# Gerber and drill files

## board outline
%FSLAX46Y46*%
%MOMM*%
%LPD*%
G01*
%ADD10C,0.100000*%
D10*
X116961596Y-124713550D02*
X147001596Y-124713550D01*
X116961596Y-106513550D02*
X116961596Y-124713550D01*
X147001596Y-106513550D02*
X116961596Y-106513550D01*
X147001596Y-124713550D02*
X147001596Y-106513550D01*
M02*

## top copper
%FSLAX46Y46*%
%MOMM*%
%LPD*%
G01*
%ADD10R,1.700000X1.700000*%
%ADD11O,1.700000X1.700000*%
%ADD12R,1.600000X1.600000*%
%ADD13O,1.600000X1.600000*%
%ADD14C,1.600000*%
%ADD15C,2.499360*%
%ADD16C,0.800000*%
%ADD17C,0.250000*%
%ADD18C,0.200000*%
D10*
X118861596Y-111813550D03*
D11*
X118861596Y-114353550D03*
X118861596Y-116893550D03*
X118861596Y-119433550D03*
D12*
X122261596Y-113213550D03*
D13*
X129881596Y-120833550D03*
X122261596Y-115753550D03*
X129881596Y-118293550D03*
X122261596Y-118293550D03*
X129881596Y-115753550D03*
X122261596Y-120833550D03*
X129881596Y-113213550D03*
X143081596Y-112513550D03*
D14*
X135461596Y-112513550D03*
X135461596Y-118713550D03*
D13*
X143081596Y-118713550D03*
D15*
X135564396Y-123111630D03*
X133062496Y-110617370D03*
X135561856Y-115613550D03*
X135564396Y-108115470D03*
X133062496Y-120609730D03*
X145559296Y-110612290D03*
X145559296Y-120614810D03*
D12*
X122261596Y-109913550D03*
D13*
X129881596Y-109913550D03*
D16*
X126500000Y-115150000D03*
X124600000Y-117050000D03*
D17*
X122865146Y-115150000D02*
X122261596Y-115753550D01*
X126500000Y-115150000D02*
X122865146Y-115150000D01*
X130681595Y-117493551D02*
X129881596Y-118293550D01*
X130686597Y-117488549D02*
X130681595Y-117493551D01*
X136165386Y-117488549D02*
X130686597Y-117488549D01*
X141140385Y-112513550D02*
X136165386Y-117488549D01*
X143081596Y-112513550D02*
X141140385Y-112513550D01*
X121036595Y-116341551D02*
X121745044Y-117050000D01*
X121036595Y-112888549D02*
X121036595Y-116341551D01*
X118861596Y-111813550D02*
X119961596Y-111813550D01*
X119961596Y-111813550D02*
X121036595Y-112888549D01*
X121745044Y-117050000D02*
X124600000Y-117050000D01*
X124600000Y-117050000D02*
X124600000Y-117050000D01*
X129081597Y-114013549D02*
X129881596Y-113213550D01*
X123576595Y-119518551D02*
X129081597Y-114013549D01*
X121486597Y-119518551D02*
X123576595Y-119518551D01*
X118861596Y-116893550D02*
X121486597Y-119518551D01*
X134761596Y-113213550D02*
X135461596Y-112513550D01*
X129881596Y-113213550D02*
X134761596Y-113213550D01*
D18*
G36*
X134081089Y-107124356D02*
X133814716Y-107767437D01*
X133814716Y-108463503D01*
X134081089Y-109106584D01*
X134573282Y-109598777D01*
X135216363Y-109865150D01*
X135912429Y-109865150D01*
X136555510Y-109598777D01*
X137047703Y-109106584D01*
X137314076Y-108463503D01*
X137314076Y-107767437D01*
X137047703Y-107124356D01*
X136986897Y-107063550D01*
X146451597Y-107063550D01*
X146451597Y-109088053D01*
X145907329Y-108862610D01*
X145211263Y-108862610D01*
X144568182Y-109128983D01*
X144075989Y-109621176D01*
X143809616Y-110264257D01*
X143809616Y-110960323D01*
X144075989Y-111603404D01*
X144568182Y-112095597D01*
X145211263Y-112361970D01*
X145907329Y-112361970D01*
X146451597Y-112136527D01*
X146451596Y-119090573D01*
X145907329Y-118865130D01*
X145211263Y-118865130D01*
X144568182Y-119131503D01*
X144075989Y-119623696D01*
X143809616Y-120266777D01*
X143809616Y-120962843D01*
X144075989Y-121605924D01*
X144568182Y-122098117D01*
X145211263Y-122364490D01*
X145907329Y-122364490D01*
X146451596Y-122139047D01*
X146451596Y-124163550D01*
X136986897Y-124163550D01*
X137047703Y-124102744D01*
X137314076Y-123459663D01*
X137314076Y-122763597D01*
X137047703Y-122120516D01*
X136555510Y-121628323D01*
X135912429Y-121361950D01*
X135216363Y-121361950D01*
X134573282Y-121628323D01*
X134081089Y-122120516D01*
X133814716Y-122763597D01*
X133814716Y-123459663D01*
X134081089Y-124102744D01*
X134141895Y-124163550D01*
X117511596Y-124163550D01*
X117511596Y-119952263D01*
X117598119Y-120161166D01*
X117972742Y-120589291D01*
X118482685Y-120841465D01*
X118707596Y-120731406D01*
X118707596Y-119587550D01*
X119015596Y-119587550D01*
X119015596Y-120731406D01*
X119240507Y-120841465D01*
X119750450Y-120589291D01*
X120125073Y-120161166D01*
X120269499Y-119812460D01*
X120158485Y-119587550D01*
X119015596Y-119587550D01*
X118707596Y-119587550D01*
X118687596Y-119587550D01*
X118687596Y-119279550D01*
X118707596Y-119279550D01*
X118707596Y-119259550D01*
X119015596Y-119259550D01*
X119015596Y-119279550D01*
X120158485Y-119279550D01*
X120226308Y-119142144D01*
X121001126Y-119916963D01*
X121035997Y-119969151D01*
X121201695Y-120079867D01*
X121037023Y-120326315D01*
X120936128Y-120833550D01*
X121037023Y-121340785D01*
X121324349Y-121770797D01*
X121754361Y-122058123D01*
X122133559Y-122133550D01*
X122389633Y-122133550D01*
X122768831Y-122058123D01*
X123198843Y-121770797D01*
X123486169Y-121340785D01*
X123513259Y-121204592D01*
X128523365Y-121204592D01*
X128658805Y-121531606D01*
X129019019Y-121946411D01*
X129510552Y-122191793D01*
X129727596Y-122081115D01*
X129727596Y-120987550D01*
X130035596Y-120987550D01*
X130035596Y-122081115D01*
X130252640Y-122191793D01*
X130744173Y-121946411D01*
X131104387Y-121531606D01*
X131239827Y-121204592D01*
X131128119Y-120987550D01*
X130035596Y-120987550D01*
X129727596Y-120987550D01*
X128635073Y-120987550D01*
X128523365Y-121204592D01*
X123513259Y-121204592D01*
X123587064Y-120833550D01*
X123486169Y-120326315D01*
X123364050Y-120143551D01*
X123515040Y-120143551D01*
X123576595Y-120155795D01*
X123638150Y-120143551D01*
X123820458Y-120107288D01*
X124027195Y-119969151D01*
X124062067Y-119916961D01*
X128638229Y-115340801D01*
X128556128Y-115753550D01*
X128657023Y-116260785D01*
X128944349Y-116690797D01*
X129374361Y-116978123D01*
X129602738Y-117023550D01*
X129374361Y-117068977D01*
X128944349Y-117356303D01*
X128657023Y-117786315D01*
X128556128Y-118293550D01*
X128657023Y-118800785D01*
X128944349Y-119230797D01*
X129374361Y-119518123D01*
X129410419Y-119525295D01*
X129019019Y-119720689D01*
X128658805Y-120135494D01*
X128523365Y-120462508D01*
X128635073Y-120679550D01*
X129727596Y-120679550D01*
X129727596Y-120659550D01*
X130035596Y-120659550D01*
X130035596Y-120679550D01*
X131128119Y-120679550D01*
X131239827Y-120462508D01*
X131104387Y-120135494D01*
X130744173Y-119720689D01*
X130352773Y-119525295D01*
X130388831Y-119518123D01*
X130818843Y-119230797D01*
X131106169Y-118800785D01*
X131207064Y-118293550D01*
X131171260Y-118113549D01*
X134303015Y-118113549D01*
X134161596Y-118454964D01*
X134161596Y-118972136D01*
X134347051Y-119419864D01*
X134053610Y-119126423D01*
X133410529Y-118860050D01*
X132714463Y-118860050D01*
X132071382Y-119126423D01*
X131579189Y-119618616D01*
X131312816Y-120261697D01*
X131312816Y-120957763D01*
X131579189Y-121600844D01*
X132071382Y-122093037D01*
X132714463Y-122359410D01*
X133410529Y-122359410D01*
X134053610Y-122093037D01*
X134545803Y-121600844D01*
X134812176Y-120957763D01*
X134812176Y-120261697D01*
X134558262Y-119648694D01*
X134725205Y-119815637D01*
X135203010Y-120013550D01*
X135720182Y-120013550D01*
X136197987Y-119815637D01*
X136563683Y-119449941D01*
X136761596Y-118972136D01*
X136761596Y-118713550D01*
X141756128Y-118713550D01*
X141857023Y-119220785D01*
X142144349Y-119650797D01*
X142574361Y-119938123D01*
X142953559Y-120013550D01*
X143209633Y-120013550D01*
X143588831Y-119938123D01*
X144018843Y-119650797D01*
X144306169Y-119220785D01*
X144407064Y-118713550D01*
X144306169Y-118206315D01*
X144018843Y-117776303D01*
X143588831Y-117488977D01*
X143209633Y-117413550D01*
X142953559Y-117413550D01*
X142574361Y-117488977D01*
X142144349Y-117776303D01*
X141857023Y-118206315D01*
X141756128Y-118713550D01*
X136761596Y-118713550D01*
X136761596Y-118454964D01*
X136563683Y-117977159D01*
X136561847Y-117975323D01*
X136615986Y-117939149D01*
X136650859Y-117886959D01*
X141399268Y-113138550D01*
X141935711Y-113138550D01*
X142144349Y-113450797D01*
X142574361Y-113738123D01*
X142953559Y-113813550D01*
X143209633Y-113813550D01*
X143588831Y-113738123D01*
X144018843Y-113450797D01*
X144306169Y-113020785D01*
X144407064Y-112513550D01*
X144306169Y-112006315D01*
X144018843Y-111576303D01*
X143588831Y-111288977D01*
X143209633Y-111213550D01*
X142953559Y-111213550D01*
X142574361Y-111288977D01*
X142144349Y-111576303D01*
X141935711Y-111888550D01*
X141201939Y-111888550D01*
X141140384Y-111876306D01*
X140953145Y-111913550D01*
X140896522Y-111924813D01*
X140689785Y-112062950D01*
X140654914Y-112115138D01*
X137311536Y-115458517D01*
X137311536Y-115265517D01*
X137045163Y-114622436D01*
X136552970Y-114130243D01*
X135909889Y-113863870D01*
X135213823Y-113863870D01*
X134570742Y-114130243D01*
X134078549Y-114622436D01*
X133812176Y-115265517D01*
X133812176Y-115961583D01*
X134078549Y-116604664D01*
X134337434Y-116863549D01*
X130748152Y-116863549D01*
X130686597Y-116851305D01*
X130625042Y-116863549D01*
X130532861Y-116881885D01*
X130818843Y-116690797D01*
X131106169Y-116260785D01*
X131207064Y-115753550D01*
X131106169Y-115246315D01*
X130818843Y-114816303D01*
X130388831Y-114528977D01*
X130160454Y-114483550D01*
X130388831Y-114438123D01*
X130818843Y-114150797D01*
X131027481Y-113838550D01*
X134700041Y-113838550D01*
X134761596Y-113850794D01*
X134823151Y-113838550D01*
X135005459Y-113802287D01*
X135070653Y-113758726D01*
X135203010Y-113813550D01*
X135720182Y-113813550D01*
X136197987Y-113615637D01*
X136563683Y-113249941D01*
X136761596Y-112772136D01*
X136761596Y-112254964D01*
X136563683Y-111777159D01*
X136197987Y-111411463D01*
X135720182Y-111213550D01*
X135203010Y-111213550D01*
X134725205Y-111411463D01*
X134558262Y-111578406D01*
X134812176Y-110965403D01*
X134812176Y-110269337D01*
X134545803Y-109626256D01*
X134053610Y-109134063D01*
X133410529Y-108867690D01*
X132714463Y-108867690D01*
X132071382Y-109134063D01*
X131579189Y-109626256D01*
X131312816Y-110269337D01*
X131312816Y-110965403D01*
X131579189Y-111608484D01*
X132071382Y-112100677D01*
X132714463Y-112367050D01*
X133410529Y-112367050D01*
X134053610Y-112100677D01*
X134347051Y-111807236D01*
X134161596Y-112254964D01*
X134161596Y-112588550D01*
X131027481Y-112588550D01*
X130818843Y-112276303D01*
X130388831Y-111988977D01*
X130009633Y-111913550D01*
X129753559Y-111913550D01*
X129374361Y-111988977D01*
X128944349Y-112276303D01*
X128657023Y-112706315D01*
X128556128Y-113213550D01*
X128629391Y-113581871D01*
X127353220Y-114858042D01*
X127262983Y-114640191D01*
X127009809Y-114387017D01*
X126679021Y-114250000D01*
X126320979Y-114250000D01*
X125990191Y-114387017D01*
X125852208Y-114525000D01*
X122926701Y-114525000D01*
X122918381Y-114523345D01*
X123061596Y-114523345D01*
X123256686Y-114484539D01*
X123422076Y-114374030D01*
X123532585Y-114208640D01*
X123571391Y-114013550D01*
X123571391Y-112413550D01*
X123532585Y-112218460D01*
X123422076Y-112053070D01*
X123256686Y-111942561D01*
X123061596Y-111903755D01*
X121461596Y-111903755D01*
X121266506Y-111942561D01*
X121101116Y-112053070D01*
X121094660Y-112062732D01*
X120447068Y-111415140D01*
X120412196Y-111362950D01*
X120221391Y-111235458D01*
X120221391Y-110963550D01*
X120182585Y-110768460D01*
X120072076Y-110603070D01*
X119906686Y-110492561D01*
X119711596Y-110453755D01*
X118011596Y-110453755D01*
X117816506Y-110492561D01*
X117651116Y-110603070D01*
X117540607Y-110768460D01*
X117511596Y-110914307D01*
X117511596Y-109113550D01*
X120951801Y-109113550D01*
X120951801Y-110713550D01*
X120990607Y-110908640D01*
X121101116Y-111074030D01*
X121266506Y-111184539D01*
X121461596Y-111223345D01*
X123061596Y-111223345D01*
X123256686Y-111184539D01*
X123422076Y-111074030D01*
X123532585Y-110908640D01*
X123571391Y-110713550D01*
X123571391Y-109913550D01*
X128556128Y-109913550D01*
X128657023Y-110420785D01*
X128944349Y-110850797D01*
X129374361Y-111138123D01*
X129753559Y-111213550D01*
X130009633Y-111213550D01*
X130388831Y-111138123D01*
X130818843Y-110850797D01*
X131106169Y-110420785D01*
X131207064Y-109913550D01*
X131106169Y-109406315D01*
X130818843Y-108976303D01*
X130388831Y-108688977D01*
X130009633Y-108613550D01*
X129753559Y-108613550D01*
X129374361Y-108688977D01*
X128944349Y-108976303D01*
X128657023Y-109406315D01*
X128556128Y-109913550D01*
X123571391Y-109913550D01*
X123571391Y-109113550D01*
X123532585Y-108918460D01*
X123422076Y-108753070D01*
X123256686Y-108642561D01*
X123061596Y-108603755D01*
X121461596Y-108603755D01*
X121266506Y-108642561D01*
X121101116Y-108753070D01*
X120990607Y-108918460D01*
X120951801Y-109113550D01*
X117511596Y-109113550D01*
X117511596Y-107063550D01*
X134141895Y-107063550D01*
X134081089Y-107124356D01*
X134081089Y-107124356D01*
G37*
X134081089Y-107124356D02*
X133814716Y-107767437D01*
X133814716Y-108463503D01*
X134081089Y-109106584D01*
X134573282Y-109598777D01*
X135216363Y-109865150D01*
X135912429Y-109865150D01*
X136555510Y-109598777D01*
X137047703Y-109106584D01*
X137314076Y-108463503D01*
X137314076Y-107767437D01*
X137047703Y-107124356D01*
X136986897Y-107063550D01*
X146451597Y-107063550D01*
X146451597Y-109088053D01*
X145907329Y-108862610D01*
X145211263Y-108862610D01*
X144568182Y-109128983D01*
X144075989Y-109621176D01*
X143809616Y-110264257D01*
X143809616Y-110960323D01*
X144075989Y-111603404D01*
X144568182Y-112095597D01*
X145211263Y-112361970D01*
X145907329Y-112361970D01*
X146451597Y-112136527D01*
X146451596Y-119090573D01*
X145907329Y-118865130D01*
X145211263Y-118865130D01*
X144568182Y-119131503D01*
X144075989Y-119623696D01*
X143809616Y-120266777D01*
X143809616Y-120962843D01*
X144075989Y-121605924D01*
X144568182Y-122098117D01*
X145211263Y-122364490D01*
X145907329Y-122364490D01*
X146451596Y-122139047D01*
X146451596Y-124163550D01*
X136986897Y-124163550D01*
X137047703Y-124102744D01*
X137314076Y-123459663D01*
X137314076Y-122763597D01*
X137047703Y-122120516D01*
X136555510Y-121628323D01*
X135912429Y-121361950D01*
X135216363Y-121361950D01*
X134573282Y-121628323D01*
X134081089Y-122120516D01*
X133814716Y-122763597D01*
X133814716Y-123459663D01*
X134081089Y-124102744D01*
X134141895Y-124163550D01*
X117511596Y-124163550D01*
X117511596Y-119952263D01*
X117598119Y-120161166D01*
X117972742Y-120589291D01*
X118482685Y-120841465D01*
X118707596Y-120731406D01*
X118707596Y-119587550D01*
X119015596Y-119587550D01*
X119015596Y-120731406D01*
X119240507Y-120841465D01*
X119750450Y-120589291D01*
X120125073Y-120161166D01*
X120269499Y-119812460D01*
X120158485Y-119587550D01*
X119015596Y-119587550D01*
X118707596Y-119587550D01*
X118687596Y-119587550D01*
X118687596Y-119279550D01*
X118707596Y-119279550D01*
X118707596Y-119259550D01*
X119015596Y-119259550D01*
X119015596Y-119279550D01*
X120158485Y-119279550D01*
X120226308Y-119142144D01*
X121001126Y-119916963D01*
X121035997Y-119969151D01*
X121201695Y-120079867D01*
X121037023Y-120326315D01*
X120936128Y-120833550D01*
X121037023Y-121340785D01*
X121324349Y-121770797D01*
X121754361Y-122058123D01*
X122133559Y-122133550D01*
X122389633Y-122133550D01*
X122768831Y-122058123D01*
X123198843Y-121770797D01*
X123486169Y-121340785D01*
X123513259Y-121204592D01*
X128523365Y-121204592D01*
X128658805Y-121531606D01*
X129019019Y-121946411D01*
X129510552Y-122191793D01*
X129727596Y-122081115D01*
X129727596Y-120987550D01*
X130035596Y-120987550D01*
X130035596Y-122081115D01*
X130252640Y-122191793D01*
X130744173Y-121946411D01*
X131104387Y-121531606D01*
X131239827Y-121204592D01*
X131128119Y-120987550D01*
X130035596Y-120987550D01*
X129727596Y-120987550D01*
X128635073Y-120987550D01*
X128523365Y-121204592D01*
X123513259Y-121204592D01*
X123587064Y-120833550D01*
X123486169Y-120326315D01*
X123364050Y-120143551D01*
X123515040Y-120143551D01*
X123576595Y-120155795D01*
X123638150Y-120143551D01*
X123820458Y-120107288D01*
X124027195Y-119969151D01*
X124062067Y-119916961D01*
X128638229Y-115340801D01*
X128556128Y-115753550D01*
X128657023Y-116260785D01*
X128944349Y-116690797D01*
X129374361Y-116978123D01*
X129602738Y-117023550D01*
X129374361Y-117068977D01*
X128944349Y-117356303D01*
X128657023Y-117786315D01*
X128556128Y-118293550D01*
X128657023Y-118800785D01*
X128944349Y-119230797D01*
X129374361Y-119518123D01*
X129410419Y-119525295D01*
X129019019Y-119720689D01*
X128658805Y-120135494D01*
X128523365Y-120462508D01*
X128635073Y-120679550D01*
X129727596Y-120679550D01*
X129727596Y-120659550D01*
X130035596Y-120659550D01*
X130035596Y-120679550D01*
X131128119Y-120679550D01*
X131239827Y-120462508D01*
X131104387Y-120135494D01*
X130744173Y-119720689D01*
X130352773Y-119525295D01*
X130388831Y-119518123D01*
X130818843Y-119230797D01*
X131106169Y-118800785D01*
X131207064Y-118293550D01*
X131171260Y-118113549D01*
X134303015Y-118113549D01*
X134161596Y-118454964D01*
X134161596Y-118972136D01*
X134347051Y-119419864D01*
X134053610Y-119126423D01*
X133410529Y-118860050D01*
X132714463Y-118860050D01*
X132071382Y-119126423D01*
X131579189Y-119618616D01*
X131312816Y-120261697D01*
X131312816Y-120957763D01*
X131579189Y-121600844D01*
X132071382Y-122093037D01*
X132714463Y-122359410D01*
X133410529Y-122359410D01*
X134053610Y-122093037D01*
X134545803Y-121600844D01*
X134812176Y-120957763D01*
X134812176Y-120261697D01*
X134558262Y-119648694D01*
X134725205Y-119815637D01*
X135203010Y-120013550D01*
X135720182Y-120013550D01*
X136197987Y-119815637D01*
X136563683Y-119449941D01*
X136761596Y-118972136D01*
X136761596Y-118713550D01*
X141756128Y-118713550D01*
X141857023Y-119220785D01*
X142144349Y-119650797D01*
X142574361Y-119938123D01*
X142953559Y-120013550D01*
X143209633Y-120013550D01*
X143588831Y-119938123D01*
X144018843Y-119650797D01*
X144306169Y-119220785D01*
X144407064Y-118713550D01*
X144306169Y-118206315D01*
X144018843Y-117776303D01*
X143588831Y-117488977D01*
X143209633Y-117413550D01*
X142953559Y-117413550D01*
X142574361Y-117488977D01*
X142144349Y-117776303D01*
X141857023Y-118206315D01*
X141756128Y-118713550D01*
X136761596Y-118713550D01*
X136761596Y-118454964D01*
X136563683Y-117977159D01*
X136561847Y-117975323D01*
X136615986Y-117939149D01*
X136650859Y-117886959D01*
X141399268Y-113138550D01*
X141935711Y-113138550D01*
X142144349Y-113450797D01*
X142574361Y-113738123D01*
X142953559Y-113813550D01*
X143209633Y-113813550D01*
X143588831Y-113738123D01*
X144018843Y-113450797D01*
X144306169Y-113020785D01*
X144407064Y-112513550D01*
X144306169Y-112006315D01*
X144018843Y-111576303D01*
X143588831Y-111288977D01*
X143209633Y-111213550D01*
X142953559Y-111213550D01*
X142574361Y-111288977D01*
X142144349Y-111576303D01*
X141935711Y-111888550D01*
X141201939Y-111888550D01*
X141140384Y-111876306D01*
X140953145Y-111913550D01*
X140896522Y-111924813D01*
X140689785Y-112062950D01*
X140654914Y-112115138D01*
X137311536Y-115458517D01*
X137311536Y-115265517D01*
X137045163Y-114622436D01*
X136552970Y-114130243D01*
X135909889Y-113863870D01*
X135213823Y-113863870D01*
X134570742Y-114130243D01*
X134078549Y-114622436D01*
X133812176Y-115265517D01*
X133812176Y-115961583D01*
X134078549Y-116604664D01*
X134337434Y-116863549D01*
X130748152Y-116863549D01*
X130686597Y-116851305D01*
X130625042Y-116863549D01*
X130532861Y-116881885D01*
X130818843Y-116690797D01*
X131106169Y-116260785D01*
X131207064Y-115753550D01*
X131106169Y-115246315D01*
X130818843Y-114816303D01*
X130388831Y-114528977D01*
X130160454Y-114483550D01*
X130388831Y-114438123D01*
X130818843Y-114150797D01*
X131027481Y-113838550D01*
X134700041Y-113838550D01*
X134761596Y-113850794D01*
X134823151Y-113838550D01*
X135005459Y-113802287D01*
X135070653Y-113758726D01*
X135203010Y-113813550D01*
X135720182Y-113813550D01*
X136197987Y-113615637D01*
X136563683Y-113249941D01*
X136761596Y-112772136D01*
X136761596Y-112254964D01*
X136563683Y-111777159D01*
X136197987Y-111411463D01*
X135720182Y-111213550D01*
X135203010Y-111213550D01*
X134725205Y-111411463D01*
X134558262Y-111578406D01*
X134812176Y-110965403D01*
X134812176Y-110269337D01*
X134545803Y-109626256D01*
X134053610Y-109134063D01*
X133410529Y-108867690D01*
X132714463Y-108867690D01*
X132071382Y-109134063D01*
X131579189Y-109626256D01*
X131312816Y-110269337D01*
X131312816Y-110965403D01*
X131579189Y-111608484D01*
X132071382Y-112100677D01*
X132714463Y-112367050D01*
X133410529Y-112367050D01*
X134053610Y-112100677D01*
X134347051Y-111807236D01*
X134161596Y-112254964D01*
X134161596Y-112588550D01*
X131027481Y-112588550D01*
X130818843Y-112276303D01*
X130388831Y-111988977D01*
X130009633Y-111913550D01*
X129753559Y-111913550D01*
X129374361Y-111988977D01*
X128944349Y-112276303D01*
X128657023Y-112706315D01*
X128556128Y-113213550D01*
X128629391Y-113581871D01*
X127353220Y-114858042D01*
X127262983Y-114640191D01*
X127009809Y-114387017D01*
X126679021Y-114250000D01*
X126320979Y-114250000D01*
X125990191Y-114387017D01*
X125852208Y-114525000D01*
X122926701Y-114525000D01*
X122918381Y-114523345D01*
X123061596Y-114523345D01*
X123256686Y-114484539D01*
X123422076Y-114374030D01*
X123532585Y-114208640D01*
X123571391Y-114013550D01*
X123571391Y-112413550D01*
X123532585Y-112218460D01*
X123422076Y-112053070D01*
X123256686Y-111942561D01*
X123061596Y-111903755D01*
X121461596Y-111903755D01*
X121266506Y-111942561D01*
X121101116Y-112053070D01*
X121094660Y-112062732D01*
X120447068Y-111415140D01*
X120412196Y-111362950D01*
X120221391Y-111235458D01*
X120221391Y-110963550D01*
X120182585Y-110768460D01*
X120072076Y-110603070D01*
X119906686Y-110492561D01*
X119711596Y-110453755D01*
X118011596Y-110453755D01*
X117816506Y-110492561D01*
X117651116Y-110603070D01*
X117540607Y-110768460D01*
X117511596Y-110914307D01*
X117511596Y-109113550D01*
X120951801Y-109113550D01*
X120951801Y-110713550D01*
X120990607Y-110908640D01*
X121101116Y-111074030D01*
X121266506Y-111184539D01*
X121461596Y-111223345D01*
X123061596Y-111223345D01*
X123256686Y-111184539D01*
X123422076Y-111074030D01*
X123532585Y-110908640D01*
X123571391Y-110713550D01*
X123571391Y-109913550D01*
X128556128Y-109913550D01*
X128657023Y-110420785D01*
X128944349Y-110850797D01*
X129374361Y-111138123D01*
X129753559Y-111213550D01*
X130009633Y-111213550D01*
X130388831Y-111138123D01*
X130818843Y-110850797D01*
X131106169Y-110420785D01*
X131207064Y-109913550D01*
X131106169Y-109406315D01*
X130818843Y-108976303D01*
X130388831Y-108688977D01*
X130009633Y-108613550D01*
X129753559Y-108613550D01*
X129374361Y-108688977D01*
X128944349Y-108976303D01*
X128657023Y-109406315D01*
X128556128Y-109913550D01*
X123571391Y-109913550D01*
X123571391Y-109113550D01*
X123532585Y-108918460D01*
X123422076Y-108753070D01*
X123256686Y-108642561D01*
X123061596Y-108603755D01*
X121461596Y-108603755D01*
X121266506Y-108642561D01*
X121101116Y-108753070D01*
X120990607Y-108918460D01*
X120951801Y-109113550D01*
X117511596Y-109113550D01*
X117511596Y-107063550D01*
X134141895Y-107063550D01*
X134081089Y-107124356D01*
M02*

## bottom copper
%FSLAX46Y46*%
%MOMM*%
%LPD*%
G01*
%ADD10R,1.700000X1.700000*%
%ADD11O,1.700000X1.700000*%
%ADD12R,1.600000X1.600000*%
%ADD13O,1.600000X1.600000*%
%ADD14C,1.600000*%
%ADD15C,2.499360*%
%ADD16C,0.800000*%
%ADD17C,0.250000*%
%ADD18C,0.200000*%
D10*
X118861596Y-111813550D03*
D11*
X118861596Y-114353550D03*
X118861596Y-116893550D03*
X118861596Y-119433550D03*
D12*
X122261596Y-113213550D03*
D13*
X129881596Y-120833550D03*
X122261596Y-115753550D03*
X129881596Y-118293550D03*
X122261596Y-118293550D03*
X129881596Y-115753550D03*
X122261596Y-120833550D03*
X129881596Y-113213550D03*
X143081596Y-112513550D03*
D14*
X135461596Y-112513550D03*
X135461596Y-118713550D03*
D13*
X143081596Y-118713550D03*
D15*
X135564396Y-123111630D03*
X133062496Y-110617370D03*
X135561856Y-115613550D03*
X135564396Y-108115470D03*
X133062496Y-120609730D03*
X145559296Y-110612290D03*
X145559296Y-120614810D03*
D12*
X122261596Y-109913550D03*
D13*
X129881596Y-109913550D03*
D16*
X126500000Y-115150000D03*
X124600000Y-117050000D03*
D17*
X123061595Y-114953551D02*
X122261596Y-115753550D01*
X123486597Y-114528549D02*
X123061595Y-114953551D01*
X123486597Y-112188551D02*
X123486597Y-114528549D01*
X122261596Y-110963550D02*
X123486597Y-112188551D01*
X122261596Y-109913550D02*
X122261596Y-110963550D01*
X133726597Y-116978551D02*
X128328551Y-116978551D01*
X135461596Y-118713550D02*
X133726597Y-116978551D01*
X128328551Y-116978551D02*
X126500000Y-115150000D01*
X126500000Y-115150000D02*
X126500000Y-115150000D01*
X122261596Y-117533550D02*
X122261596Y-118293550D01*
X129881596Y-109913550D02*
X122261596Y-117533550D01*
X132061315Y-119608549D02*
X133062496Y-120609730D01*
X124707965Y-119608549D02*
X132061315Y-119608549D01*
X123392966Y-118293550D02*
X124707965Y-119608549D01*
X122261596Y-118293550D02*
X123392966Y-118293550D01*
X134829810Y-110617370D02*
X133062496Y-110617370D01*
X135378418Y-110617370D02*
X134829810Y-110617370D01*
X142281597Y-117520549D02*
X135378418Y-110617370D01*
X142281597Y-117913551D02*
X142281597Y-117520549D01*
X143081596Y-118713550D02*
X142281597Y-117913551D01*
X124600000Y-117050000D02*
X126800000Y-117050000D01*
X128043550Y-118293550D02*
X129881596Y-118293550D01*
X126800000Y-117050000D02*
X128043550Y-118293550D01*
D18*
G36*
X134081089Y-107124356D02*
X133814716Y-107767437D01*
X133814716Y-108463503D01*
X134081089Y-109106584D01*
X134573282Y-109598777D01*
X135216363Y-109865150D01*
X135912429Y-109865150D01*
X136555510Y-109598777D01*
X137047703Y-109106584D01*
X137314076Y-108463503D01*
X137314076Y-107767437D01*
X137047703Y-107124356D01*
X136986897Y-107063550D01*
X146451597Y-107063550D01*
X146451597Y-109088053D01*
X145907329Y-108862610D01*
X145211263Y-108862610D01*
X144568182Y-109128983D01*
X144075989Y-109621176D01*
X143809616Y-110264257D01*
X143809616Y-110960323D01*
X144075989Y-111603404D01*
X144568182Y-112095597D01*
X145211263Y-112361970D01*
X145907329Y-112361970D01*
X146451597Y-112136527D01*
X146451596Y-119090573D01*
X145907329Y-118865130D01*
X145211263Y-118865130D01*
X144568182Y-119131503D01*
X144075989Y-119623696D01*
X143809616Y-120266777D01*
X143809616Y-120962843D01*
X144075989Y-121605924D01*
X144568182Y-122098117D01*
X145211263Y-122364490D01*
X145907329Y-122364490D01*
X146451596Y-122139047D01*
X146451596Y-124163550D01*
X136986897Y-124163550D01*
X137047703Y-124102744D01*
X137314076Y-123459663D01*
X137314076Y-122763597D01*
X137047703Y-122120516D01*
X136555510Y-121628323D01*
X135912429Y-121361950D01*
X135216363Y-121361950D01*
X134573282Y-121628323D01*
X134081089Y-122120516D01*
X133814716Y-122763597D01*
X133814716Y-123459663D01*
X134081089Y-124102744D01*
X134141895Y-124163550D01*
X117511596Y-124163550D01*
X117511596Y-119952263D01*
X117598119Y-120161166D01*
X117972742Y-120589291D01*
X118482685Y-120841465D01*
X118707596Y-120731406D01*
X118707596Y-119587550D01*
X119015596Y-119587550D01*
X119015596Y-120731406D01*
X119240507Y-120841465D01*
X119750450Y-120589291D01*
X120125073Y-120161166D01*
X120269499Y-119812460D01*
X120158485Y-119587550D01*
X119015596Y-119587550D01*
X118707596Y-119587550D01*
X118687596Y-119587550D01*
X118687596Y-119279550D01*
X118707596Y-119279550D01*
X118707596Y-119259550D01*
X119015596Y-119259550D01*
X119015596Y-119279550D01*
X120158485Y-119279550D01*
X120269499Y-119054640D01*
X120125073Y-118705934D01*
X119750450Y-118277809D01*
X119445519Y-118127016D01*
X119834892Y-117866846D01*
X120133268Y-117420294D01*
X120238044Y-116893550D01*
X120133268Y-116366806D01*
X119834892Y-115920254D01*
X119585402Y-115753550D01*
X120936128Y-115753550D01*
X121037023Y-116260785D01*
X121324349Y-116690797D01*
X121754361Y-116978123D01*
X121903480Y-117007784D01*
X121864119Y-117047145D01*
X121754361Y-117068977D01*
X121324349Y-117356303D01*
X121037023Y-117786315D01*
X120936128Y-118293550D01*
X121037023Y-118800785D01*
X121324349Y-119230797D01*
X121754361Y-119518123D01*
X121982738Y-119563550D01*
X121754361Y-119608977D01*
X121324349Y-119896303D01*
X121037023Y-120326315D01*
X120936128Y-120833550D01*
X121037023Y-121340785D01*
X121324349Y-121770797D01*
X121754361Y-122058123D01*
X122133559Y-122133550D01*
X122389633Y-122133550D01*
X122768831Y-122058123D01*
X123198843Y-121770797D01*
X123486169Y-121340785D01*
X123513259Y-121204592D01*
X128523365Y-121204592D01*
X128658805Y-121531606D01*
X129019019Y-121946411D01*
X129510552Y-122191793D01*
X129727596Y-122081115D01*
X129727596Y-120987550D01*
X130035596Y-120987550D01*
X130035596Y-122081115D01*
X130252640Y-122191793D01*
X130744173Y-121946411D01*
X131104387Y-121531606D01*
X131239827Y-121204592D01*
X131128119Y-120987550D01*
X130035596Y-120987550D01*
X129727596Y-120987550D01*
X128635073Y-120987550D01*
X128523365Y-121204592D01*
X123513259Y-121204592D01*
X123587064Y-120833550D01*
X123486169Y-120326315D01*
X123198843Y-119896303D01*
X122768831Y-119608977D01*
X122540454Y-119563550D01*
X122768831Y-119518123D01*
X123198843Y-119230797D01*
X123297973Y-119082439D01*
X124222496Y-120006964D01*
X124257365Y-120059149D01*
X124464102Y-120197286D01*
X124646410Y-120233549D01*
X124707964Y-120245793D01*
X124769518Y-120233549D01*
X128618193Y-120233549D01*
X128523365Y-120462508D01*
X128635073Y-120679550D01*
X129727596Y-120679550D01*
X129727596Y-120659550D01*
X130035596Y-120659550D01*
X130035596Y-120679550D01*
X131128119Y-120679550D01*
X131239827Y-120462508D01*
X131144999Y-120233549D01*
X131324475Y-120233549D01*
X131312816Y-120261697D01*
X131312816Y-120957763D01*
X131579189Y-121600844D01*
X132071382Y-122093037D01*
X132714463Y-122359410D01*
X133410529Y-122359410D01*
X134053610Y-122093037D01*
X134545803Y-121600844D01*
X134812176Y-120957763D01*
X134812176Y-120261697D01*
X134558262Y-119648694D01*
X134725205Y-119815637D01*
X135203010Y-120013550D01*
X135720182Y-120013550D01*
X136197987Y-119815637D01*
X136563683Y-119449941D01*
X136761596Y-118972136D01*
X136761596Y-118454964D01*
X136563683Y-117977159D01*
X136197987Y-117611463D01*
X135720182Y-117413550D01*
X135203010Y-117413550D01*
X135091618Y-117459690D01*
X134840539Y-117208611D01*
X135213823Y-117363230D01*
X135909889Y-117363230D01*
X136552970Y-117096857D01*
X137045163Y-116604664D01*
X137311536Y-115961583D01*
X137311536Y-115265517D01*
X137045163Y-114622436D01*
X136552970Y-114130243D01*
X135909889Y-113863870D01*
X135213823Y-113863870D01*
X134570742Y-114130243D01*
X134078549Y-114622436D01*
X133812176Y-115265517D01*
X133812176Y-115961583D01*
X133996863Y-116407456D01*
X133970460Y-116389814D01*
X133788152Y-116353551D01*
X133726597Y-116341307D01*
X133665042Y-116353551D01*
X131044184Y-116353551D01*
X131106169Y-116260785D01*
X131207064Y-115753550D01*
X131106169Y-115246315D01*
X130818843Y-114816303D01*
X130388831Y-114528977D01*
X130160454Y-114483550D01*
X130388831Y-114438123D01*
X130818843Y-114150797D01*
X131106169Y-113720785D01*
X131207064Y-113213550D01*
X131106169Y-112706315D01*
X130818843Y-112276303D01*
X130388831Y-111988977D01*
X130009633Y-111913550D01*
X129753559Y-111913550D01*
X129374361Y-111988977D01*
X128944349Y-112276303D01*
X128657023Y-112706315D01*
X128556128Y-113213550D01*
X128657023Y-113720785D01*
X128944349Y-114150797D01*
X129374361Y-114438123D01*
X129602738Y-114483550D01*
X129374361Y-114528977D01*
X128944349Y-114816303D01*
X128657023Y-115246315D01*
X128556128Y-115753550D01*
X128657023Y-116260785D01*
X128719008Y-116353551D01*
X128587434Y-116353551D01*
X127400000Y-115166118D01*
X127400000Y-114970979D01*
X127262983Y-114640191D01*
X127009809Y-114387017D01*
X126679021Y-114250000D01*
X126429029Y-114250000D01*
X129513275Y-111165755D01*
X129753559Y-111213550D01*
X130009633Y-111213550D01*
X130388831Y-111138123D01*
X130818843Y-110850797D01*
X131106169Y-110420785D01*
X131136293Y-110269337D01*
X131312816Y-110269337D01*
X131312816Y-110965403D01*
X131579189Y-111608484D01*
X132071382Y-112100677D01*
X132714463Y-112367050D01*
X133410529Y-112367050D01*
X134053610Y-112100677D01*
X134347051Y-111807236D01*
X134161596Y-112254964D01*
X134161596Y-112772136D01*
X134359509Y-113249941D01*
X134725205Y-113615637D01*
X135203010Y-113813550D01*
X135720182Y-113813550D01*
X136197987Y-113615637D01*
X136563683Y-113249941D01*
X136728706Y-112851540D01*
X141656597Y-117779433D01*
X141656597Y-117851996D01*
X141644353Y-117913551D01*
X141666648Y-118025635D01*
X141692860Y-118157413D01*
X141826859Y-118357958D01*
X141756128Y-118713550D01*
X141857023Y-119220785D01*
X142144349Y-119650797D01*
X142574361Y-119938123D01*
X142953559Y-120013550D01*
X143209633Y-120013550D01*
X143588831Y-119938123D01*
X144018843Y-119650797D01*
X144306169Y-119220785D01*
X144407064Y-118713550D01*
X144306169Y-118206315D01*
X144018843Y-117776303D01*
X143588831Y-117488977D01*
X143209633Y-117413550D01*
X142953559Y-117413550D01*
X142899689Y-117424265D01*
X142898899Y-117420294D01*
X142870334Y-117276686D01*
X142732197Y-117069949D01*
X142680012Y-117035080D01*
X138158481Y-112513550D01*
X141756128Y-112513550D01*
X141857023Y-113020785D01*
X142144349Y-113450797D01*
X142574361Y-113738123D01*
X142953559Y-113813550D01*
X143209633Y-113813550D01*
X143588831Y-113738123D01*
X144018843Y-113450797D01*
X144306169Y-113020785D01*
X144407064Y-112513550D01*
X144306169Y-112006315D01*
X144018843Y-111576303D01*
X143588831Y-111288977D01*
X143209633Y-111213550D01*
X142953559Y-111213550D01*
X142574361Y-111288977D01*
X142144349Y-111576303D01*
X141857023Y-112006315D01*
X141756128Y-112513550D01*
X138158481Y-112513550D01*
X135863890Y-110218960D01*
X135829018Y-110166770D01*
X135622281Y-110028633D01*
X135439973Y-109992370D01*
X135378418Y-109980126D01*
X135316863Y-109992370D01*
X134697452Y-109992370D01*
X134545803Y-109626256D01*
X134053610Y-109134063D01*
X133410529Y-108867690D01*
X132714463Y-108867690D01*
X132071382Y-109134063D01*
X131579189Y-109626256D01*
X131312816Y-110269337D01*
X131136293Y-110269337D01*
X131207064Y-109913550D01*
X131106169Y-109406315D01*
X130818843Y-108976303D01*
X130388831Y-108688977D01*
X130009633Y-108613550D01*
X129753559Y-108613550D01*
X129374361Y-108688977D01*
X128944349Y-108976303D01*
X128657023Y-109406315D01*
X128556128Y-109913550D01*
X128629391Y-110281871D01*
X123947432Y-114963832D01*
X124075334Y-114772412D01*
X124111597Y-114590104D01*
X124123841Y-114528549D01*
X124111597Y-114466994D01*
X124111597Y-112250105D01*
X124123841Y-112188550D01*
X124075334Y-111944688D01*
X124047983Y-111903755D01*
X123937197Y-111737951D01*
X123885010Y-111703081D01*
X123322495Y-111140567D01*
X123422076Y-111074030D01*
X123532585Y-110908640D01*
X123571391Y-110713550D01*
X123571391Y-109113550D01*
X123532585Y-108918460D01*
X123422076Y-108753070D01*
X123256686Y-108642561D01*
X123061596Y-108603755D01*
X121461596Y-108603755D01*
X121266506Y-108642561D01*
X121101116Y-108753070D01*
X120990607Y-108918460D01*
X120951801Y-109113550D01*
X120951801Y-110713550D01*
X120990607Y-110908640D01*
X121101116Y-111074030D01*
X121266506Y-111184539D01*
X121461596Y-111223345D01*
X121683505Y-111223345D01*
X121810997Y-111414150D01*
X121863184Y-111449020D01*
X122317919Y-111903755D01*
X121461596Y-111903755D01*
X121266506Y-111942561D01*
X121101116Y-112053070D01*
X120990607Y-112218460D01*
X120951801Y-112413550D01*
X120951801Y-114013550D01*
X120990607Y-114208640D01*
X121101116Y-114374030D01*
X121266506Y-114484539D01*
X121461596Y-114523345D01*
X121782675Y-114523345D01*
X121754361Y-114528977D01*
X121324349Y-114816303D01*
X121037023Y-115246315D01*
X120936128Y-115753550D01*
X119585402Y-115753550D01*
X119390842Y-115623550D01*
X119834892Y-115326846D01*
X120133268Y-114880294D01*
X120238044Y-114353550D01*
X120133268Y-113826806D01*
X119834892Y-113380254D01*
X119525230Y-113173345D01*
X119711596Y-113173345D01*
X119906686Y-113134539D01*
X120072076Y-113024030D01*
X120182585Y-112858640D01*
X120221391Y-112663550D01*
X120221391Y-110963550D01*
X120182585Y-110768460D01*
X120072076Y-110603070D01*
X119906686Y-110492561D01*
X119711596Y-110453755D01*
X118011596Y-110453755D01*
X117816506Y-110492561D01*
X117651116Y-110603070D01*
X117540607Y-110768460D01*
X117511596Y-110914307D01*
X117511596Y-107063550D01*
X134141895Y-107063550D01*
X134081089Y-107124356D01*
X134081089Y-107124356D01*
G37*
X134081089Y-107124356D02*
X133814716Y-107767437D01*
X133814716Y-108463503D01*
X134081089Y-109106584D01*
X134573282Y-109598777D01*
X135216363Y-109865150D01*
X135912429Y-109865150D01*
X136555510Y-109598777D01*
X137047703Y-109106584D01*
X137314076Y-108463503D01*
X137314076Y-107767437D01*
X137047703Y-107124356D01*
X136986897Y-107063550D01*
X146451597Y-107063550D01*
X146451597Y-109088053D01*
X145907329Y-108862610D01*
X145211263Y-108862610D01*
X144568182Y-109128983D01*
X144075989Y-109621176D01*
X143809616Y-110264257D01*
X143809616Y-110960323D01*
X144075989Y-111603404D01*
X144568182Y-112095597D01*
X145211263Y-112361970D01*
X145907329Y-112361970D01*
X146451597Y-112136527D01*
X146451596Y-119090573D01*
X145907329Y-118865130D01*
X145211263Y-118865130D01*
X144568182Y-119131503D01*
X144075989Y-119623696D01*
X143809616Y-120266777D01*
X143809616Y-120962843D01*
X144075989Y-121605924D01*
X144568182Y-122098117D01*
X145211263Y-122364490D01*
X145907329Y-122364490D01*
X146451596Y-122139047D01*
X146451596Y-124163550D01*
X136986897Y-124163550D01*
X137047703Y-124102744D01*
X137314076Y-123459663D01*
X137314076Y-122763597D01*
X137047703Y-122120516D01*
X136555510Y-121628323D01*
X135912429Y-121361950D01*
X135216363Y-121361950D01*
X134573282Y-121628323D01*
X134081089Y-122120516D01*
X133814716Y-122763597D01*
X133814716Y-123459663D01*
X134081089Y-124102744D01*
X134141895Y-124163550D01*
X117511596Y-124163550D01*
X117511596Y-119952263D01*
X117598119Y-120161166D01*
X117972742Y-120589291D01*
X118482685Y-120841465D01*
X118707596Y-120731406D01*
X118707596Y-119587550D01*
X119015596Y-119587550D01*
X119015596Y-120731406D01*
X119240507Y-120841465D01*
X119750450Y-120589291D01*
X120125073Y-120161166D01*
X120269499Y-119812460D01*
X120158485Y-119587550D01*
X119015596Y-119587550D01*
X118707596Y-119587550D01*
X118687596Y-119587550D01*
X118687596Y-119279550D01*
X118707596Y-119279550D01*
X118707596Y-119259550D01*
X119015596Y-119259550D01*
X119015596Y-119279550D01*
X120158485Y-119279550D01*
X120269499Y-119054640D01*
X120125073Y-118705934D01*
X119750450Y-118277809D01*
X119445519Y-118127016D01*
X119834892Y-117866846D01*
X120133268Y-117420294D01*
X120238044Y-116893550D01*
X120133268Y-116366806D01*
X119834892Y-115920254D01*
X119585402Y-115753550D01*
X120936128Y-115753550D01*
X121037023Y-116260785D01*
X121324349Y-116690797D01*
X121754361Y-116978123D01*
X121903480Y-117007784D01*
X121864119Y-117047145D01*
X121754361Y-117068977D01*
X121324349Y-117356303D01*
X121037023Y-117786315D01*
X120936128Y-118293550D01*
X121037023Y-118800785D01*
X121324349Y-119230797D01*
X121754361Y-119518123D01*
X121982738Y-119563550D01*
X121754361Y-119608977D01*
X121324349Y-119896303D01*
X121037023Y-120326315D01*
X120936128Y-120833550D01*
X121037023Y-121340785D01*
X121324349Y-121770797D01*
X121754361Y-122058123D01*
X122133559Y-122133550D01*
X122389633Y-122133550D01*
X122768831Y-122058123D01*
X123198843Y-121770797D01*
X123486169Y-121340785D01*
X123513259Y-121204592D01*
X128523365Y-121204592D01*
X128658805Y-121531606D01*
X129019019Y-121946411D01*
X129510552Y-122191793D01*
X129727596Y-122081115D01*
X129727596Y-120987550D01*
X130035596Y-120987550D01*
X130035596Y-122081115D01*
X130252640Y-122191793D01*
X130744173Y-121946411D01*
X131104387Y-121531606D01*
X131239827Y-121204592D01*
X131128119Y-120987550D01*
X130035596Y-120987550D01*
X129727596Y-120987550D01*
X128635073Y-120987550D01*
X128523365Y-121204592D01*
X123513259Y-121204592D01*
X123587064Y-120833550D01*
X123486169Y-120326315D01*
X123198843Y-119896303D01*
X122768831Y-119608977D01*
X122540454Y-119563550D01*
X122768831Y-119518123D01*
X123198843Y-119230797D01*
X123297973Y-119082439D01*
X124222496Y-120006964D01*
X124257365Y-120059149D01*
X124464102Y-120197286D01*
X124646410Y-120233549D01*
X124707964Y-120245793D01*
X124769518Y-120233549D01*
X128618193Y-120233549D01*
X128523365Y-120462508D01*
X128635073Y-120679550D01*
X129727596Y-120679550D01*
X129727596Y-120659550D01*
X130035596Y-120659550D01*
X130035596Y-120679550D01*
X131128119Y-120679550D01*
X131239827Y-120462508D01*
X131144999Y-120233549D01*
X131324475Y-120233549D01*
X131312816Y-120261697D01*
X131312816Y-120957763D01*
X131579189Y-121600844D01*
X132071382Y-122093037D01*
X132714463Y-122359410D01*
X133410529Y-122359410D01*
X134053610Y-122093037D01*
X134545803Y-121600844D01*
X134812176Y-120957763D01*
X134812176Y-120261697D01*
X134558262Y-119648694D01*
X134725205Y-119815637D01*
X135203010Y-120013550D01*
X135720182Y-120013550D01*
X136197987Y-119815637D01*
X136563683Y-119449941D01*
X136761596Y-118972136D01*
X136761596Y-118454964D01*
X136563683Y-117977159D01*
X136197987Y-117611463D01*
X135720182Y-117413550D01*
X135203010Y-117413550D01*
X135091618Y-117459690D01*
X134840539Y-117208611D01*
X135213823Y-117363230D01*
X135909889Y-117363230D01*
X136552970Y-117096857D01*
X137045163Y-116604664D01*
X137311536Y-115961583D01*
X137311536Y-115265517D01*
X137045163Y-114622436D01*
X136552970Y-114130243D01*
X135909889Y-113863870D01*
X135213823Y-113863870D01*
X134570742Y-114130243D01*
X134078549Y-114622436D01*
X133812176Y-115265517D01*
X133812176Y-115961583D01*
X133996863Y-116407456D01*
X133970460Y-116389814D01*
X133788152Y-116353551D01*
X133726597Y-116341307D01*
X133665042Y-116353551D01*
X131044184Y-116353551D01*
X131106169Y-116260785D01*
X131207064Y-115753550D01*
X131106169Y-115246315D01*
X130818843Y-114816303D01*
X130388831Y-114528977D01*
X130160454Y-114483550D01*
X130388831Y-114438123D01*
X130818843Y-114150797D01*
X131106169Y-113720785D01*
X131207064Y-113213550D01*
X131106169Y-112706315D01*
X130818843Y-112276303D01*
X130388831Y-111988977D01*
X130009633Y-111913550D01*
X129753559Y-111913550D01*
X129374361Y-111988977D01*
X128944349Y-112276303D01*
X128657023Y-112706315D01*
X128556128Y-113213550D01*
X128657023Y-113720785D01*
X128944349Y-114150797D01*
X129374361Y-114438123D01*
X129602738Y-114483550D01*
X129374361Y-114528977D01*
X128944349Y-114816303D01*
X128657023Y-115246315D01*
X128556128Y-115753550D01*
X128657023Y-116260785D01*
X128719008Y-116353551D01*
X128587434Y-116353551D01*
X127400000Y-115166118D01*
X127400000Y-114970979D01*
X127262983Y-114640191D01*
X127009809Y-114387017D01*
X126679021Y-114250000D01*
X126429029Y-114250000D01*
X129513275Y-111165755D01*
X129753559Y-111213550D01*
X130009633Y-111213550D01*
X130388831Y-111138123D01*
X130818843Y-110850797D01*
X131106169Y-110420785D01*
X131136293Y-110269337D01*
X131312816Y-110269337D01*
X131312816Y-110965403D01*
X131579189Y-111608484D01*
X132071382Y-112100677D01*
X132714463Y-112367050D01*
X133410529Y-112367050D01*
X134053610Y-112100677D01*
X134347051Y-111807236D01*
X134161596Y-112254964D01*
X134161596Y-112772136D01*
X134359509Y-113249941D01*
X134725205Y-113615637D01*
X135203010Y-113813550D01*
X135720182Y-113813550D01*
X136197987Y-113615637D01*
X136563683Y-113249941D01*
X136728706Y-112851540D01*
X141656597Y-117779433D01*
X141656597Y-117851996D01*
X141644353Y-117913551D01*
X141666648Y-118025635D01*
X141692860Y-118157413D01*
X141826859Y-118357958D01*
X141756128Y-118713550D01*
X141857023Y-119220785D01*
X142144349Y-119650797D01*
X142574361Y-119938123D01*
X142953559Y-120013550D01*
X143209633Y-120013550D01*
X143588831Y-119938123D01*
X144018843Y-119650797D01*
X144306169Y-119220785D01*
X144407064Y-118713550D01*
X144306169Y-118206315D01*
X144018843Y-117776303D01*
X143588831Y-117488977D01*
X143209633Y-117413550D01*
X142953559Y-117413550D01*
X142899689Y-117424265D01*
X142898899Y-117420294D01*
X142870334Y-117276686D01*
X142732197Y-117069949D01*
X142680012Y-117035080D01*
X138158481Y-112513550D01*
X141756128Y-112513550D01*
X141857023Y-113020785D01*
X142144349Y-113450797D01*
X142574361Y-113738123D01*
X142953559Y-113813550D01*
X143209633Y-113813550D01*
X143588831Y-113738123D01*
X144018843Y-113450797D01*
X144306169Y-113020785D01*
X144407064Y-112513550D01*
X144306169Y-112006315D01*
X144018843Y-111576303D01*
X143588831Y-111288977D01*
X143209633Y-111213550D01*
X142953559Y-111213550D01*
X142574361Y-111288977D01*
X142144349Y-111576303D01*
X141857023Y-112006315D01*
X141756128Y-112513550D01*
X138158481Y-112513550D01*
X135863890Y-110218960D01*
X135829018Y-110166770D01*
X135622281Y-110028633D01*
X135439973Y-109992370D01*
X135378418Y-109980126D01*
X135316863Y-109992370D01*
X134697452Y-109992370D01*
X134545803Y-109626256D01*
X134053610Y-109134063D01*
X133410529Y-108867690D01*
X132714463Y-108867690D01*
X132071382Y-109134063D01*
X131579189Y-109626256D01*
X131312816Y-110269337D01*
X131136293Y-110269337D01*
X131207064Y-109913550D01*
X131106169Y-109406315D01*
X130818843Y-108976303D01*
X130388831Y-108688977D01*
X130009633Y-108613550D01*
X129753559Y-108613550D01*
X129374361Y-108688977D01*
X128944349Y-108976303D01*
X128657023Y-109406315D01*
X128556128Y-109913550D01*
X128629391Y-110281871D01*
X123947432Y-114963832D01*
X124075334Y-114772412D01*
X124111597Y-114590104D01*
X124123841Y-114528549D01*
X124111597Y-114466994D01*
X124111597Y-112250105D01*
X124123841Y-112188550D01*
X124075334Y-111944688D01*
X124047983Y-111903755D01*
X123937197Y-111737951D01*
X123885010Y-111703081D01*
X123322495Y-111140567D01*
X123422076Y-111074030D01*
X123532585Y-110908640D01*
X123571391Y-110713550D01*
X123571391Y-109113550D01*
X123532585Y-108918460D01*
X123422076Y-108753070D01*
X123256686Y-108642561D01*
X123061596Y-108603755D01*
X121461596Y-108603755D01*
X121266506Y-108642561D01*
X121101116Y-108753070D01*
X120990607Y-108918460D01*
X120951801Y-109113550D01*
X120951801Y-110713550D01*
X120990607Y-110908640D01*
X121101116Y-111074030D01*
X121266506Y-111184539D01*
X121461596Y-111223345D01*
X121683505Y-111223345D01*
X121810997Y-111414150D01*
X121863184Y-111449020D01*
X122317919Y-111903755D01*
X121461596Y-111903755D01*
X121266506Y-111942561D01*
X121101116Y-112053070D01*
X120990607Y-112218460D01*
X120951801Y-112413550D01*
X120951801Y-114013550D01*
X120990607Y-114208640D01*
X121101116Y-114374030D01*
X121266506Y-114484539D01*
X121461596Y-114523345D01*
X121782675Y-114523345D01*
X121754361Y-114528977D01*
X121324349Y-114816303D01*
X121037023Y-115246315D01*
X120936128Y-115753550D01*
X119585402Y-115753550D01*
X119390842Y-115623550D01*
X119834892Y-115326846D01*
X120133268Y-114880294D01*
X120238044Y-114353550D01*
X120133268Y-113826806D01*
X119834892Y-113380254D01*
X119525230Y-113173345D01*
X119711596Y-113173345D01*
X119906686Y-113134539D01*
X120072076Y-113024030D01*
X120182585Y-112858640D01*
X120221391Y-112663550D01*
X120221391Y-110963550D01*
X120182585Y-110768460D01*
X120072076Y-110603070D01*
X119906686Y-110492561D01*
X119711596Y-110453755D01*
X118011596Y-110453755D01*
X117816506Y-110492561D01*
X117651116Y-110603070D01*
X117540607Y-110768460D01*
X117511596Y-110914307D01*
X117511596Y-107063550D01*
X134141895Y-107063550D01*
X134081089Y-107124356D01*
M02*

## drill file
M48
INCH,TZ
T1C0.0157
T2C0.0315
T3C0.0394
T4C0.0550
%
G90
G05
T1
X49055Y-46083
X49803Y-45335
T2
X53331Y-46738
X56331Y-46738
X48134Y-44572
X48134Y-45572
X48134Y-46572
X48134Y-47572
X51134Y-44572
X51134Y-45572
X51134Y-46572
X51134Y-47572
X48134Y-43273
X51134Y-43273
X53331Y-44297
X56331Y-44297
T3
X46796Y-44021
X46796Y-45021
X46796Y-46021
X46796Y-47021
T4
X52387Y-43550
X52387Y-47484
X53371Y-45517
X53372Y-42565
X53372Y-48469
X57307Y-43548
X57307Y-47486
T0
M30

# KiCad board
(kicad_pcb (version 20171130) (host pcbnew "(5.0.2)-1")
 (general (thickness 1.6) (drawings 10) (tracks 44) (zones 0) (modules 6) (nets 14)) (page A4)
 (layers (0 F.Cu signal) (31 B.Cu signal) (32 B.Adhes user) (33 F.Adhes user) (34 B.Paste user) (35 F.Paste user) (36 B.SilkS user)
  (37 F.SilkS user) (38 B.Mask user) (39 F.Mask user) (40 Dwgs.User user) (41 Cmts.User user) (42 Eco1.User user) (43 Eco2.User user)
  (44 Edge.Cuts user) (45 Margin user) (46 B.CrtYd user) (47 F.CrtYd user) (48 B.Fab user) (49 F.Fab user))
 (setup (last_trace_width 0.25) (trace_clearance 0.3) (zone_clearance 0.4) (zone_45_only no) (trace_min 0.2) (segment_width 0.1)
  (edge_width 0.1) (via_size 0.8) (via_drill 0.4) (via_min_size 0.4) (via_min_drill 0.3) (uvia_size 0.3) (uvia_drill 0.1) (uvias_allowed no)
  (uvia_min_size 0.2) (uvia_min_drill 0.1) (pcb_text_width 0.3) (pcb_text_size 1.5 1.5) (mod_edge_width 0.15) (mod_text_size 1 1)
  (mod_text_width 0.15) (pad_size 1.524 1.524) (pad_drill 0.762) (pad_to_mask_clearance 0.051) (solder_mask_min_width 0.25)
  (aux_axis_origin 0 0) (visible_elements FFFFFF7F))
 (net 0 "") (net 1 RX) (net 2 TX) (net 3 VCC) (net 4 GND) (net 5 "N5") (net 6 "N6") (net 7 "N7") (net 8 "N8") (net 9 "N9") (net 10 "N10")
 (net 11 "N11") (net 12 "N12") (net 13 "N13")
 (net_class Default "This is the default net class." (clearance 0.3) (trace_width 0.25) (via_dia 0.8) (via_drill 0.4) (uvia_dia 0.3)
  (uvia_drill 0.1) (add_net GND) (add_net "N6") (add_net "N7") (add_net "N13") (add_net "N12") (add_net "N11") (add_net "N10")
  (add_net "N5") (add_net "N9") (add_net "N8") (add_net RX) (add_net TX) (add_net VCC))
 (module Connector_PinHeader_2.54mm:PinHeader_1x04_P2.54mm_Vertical (layer F.Cu) (at 118.861596 111.81355)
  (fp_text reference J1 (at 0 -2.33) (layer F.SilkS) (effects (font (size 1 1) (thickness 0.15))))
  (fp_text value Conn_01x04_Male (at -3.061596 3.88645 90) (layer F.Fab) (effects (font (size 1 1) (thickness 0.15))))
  (pad 1 thru_hole rect (at 0 0) (size 1.7 1.7) (drill 1) (layers *.Cu *.Mask) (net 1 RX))
  (pad 2 thru_hole oval (at 0 2.54) (size 1.7 1.7) (drill 1) (layers *.Cu *.Mask) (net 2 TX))
  (pad 3 thru_hole oval (at 0 5.08) (size 1.7 1.7) (drill 1) (layers *.Cu *.Mask) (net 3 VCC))
  (pad 4 thru_hole oval (at 0 7.62) (size 1.7 1.7) (drill 1) (layers *.Cu *.Mask) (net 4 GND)))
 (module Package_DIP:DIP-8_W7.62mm (layer F.Cu) (at 122.261596 113.21355)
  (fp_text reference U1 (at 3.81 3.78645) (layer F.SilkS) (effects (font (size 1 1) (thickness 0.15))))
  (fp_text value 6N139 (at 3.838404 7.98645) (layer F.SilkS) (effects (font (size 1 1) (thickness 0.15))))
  (pad 1 thru_hole rect (at 0 0) (size 1.6 1.6) (drill 0.8) (layers *.Cu *.Mask) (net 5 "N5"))
  (pad 5 thru_hole oval (at 7.62 7.62) (size 1.6 1.6) (drill 0.8) (layers *.Cu *.Mask) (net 4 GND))
  (pad 2 thru_hole oval (at 0 2.54) (size 1.6 1.6) (drill 0.8) (layers *.Cu *.Mask) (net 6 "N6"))
  (pad 6 thru_hole oval (at 7.62 5.08) (size 1.6 1.6) (drill 0.8) (layers *.Cu *.Mask) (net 1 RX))
  (pad 3 thru_hole oval (at 0 5.08) (size 1.6 1.6) (drill 0.8) (layers *.Cu *.Mask) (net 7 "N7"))
  (pad 7 thru_hole oval (at 7.62 2.54) (size 1.6 1.6) (drill 0.8) (layers *.Cu *.Mask) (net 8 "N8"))
  (pad 4 thru_hole oval (at 0 7.62) (size 1.6 1.6) (drill 0.8) (layers *.Cu *.Mask) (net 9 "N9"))
  (pad 8 thru_hole oval (at 7.62 0) (size 1.6 1.6) (drill 0.8) (layers *.Cu *.Mask) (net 3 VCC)))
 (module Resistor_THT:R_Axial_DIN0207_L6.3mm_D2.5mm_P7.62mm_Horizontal (layer B.Cu) (at 135.461596 112.51355)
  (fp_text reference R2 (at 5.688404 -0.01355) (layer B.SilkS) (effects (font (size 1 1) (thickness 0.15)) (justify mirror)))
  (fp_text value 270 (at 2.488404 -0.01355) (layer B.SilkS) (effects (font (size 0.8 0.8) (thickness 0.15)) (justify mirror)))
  (pad 2 thru_hole oval (at 7.62 0) (size 1.6 1.6) (drill 0.8) (layers *.Cu *.Mask) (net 1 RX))
  (pad 1 thru_hole circle (at 0 0) (size 1.6 1.6) (drill 0.8) (layers *.Cu *.Mask) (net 3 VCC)))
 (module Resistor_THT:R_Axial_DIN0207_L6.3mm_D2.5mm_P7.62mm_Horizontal (layer B.Cu) (at 135.461596 118.71355)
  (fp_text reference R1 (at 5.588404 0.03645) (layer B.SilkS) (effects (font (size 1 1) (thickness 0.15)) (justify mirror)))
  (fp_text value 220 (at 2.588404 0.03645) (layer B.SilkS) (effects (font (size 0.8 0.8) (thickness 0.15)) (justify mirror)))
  (pad 1 thru_hole circle (at 0 0) (size 1.6 1.6) (drill 0.8) (layers *.Cu *.Mask) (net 6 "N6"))
  (pad 2 thru_hole oval (at 7.62 0) (size 1.6 1.6) (drill 0.8) (layers *.Cu *.Mask) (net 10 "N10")))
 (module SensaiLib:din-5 (layer F.Cu) (at 138.561596 115.61355 90)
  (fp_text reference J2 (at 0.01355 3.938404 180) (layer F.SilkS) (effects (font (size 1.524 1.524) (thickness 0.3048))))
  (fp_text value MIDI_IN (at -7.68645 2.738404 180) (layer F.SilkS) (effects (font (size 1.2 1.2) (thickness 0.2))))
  (pad 3 thru_hole circle (at -7.49808 -2.9972 90) (size 2.49936 2.49936) (drill 1.397) (layers *.Cu *.SilkS *.Mask) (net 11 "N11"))
  (pad 4 thru_hole circle (at 4.99618 -5.4991 90) (size 2.49936 2.49936) (drill 1.397) (layers *.Cu *.SilkS *.Mask) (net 10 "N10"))
  (pad 2 thru_hole circle (at 0 -2.99974 90) (size 2.49936 2.49936) (drill 1.397) (layers *.Cu *.SilkS *.Mask) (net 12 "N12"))
  (pad 1 thru_hole circle (at 7.49808 -2.9972 90) (size 2.49936 2.49936) (drill 1.397) (layers *.Cu *.SilkS *.Mask) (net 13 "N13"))
  (pad 5 thru_hole circle (at -4.99618 -5.4991 90) (size 2.49936 2.49936) (drill 1.397) (layers *.Cu *.SilkS *.Mask) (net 7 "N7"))
  (pad "" thru_hole circle (at 5.00126 6.9977 90) (size 2.49936 2.49936) (drill 1.397) (layers *.Cu *.Mask))
  (pad "" thru_hole circle (at -5.00126 6.9977 90) (size 2.49936 2.49936) (drill 1.397) (layers *.Cu *.Mask)))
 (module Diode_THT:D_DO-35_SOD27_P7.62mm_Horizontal (layer F.Cu) (at 122.261596 109.91355)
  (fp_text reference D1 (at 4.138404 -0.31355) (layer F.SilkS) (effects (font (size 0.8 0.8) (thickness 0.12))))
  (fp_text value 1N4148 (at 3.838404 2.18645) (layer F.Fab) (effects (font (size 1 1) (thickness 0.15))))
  (pad 1 thru_hole rect (at 0 0) (size 1.6 1.6) (drill 0.8) (layers *.Cu *.Mask) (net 6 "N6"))
  (pad 2 thru_hole oval (at 7.62 0) (size 1.6 1.6) (drill 0.8) (layers *.Cu *.Mask) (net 7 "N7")))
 (gr_line (start 116.961596 124.71355) (end 147.001596 124.71355) (layer Edge.Cuts) (width 0.1))
 (gr_line (start 116.961596 106.51355) (end 116.961596 124.71355) (layer Edge.Cuts) (width 0.1))
 (gr_line (start 147.001596 106.51355) (end 116.961596 106.51355) (layer Edge.Cuts) (width 0.1))
 (gr_line (start 147.001596 124.71355) (end 147.001596 106.51355) (layer Edge.Cuts) (width 0.1))
 (segment (start 123.061595 114.953551) (end 122.261596 115.75355) (width 0.25) (layer B.Cu) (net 6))
 (segment (start 123.486597 114.528549) (end 123.061595 114.953551) (width 0.25) (layer B.Cu) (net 6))
 (segment (start 123.486597 112.188551) (end 123.486597 114.528549) (width 0.25) (layer B.Cu) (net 6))
 (segment (start 122.261596 110.96355) (end 123.486597 112.188551) (width 0.25) (layer B.Cu) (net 6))
 (segment (start 122.261596 109.91355) (end 122.261596 110.96355) (width 0.25) (layer B.Cu) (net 6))
 (segment (start 133.726597 116.978551) (end 128.328551 116.978551) (width 0.25) (layer B.Cu) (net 6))
 (segment (start 135.461596 118.71355) (end 133.726597 116.978551) (width 0.25) (layer B.Cu) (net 6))
 (segment (start 128.328551 116.978551) (end 126.5 115.15) (width 0.25) (layer B.Cu) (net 6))
 (segment (start 126.5 115.15) (end 126.5 115.15) (width 0.25) (layer B.Cu) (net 6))
 (via (at 126.5 115.15) (size 0.8) (drill 0.4) (layers F.Cu B.Cu) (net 6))
 (segment (start 122.865146 115.15) (end 122.261596 115.75355) (width 0.25) (layer F.Cu) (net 6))
 (segment (start 126.5 115.15) (end 122.865146 115.15) (width 0.25) (layer F.Cu) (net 6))
 (segment (start 122.261596 117.53355) (end 122.261596 118.29355) (width 0.25) (layer B.Cu) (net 7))
 (segment (start 129.881596 109.91355) (end 122.261596 117.53355) (width 0.25) (layer B.Cu) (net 7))
 (segment (start 132.061315 119.608549) (end 133.062496 120.60973) (width 0.25) (layer B.Cu) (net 7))
 (segment (start 124.707965 119.608549) (end 132.061315 119.608549) (width 0.25) (layer B.Cu) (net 7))
 (segment (start 123.392966 118.29355) (end 124.707965 119.608549) (width 0.25) (layer B.Cu) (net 7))
 (segment (start 122.261596 118.29355) (end 123.392966 118.29355) (width 0.25) (layer B.Cu) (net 7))
 (segment (start 134.82981 110.61737) (end 133.062496 110.61737) (width 0.25) (layer B.Cu) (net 10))
 (segment (start 135.378418 110.61737) (end 134.82981 110.61737) (width 0.25) (layer B.Cu) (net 10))
 (segment (start 142.281597 117.520549) (end 135.378418 110.61737) (width 0.25) (layer B.Cu) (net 10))
 (segment (start 142.281597 117.913551) (end 142.281597 117.520549) (width 0.25) (layer B.Cu) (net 10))
 (segment (start 143.081596 118.71355) (end 142.281597 117.913551) (width 0.25) (layer B.Cu) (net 10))
 (segment (start 130.681595 117.493551) (end 129.881596 118.29355) (width 0.25) (layer F.Cu) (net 1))
 (segment (start 130.686597 117.488549) (end 130.681595 117.493551) (width 0.25) (layer F.Cu) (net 1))
 (segment (start 136.165386 117.488549) (end 130.686597 117.488549) (width 0.25) (layer F.Cu) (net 1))
 (segment (start 141.140385 112.51355) (end 136.165386 117.488549) (width 0.25) (layer F.Cu) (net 1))
 (segment (start 143.081596 112.51355) (end 141.140385 112.51355) (width 0.25) (layer F.Cu) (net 1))
 (segment (start 121.036595 116.341551) (end 121.745044 117.05) (width 0.25) (layer F.Cu) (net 1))
 (segment (start 121.036595 112.888549) (end 121.036595 116.341551) (width 0.25) (layer F.Cu) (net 1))
 (segment (start 118.861596 111.81355) (end 119.961596 111.81355) (width 0.25) (layer F.Cu) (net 1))
 (segment (start 119.961596 111.81355) (end 121.036595 112.888549) (width 0.25) (layer F.Cu) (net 1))
 (segment (start 121.745044 117.05) (end 124.6 117.05) (width 0.25) (layer F.Cu) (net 1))
 (segment (start 124.6 117.05) (end 124.6 117.05) (width 0.25) (layer F.Cu) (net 1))
 (via (at 124.6 117.05) (size 0.8) (drill 0.4) (layers F.Cu B.Cu) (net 1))
 (segment (start 124.6 117.05) (end 126.8 117.05) (width 0.25) (layer B.Cu) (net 1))
 (segment (start 128.04355 118.29355) (end 129.881596 118.29355) (width 0.25) (layer B.Cu) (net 1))
 (segment (start 126.8 117.05) (end 128.04355 118.29355) (width 0.25) (layer B.Cu) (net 1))
 (segment (start 129.081597 114.013549) (end 129.881596 113.21355) (width 0.25) (layer F.Cu) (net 3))
 (segment (start 123.576595 119.518551) (end 129.081597 114.013549) (width 0.25) (layer F.Cu) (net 3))
 (segment (start 121.486597 119.518551) (end 123.576595 119.518551) (width 0.25) (layer F.Cu) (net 3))
 (segment (start 118.861596 116.89355) (end 121.486597 119.518551) (width 0.25) (layer F.Cu) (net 3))
 (segment (start 134.761596 113.21355) (end 135.461596 112.51355) (width 0.25) (layer F.Cu) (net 3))
 (segment (start 129.881596 113.21355) (end 134.761596 113.21355) (width 0.25) (layer F.Cu) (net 3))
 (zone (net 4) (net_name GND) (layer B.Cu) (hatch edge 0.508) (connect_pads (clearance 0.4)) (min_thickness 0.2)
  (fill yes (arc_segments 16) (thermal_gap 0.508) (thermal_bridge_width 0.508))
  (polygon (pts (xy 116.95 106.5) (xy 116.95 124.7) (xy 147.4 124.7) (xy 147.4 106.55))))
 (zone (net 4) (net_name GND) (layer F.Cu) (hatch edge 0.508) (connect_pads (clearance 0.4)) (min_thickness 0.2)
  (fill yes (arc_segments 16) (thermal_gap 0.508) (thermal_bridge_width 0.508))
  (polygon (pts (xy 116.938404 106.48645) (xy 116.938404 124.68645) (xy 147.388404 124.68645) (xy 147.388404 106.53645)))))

